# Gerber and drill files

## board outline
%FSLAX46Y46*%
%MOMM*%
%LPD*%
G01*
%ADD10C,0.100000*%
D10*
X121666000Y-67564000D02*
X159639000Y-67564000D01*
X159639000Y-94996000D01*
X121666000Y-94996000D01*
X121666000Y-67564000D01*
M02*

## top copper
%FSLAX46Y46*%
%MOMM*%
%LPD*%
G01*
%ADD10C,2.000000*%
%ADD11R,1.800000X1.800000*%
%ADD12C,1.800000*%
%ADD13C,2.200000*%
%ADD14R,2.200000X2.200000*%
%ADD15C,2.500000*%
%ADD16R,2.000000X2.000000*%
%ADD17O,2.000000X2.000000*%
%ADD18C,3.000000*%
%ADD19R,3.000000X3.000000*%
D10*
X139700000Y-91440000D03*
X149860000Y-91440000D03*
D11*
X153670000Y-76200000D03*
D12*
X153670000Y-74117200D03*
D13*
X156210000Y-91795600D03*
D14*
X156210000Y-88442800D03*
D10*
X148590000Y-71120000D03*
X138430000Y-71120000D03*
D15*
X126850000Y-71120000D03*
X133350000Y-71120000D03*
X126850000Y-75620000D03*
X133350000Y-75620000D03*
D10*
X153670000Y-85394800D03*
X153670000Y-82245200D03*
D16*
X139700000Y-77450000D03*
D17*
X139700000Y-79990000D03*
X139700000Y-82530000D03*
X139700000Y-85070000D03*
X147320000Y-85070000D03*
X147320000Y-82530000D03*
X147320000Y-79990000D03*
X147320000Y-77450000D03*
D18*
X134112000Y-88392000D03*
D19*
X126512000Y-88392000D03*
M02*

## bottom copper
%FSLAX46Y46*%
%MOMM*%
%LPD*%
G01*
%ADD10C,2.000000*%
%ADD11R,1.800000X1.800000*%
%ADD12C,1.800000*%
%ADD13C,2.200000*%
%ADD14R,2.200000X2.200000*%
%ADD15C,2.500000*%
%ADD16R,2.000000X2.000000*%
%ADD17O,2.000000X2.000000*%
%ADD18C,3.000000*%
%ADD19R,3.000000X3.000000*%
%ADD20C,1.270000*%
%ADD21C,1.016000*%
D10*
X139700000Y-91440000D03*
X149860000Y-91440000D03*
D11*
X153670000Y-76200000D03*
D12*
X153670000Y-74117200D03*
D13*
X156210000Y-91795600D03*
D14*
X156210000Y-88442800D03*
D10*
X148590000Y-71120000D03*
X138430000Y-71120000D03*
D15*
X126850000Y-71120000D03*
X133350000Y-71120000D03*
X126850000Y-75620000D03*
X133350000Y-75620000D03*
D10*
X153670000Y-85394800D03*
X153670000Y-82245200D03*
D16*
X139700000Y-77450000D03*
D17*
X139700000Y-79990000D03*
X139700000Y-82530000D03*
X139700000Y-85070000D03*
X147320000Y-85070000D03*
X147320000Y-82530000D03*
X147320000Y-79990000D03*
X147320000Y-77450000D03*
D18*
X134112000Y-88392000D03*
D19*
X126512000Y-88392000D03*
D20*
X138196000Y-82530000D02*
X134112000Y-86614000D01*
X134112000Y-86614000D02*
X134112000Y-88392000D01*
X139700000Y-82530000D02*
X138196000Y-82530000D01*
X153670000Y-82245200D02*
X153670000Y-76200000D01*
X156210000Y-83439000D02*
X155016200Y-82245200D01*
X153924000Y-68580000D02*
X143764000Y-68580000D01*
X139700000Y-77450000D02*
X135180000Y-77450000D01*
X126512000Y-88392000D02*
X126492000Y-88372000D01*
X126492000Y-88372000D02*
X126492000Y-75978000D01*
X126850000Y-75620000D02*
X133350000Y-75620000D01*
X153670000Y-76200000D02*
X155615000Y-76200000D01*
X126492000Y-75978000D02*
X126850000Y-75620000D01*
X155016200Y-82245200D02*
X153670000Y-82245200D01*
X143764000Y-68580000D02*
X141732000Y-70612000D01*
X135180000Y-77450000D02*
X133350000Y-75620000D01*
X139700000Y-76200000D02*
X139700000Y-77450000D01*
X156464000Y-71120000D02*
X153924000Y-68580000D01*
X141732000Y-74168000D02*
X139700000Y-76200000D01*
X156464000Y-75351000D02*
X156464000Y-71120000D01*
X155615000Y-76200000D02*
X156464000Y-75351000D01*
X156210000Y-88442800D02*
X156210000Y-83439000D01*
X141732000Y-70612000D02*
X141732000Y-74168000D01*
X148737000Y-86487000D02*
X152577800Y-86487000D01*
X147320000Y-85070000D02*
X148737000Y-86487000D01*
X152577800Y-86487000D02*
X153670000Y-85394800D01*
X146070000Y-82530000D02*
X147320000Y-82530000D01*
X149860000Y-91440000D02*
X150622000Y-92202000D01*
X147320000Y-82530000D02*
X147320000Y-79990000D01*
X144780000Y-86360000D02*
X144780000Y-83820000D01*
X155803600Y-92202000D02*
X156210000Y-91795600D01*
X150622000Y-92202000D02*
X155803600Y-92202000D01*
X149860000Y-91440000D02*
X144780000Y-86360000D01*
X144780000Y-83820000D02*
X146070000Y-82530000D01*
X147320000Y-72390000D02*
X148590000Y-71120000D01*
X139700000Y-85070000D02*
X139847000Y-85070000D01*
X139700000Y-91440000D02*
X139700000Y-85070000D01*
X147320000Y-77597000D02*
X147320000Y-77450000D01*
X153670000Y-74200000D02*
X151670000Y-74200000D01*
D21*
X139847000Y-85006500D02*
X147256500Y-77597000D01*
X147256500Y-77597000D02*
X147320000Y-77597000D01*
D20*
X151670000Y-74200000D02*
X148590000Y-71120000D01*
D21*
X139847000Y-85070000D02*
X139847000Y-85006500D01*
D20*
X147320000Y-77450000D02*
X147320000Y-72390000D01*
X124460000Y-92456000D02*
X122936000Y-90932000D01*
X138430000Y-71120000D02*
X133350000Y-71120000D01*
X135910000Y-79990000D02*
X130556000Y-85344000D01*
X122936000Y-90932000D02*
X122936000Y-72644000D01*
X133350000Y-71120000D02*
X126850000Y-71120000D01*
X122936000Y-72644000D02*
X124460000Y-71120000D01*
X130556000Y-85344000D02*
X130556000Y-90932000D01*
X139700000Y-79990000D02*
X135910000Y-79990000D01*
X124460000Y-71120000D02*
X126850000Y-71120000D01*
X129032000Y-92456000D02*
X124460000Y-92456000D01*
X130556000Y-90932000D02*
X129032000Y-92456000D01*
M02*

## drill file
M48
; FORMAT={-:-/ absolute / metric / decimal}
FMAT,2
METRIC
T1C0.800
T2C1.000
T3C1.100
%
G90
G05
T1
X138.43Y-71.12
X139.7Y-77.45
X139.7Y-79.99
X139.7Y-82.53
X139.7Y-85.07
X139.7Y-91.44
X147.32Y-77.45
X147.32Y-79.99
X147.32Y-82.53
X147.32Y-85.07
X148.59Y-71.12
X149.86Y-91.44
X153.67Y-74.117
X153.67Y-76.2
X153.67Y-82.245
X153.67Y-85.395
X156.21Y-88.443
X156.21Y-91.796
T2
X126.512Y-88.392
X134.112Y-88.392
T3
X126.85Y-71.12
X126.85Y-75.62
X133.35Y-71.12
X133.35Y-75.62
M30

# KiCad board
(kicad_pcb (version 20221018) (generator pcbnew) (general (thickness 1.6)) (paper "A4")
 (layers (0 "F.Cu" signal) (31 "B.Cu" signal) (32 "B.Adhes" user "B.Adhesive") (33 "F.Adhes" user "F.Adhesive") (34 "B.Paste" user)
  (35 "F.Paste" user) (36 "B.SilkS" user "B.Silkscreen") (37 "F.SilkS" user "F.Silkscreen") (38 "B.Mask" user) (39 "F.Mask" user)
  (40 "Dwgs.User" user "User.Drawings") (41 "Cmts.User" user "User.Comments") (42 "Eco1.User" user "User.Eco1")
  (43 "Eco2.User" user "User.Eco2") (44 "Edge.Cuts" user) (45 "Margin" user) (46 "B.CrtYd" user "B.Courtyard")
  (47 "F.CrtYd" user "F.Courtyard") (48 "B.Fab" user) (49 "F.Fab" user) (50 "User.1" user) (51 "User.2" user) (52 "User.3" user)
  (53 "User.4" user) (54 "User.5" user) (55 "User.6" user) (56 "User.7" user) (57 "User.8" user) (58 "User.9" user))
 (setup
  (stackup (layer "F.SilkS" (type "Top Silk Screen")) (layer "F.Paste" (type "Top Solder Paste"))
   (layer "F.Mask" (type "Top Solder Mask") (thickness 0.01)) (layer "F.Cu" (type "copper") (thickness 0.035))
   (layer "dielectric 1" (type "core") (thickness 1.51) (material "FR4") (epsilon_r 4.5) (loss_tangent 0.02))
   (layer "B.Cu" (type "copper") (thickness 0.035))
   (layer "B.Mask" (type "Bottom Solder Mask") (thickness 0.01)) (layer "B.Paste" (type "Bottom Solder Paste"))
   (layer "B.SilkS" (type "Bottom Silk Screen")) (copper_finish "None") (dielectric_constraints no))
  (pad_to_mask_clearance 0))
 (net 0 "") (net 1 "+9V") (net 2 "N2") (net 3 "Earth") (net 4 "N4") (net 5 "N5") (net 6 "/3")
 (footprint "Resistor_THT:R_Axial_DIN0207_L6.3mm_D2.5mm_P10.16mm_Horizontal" (layer "F.Cu") (at 139.7 91.44)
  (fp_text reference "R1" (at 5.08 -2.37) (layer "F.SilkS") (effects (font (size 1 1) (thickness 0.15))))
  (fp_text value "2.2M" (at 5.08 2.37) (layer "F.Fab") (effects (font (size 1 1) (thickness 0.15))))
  (pad "1" thru_hole circle (at 0 0) (size 2 2) (drill 0.8) (layers "*.Cu" "*.Mask") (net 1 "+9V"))
  (pad "2" thru_hole circle (at 10.16 0) (size 2 2) (drill 0.8) (layers "*.Cu" "*.Mask") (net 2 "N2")))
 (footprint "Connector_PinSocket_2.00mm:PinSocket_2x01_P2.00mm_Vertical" (layer "F.Cu") (at 153.67 76.2 -90)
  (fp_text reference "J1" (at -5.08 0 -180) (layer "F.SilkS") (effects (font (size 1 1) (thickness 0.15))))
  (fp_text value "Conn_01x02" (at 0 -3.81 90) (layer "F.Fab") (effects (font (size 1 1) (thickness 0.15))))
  (pad "1" thru_hole rect (at 0 0 270) (size 1.8 1.8) (drill 0.8) (layers "*.Cu" "*.Mask") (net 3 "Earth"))
  (pad "2" thru_hole circle (at -2.0828 0 270) (size 1.8 1.8) (drill 0.8) (layers "*.Cu" "*.Mask") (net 1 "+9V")))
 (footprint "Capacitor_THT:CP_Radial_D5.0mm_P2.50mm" (layer "F.Cu") (at 156.21 91.44 90)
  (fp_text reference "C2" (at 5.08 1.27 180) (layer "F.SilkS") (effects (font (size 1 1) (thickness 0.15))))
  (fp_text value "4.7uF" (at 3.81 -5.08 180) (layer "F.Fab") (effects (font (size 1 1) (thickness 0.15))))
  (pad "1" thru_hole circle (at -0.3556 0 90) (size 2.2 2.2) (drill 0.8) (layers "*.Cu" "*.Mask") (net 2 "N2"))
  (pad "2" thru_hole rect (at 2.9972 0 90) (size 2.2 2.2) (drill 0.8) (layers "*.Cu" "*.Mask") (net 3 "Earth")))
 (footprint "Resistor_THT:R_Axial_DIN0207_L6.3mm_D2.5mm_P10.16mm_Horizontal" (layer "F.Cu") (at 148.59 71.12 180)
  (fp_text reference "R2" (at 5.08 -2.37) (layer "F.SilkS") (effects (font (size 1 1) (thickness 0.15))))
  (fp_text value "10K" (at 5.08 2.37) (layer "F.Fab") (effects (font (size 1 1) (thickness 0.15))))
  (pad "1" thru_hole circle (at 0 0 180) (size 2 2) (drill 0.8) (layers "*.Cu" "*.Mask") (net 1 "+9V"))
  (pad "2" thru_hole circle (at 10.16 0 180) (size 2 2) (drill 0.8) (layers "*.Cu" "*.Mask") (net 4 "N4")))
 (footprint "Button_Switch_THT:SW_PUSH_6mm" (layer "F.Cu") (at 126.85 71.12)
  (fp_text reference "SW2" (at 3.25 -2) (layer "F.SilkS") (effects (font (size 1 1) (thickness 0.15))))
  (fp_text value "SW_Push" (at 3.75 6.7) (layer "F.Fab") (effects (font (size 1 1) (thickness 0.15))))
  (pad "1" thru_hole circle (at 0 0 90) (size 2.5 2.5) (drill 1.1) (layers "*.Cu" "*.Mask") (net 4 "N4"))
  (pad "1" thru_hole circle (at 6.5 0 90) (size 2.5 2.5) (drill 1.1) (layers "*.Cu" "*.Mask") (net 4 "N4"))
  (pad "2" thru_hole circle (at 0 4.5 90) (size 2.5 2.5) (drill 1.1) (layers "*.Cu" "*.Mask") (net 3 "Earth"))
  (pad "2" thru_hole circle (at 6.5 4.5 90) (size 2.5 2.5) (drill 1.1) (layers "*.Cu" "*.Mask") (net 3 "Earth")))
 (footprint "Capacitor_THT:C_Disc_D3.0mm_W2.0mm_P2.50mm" (layer "F.Cu") (at 153.67 85.09 90)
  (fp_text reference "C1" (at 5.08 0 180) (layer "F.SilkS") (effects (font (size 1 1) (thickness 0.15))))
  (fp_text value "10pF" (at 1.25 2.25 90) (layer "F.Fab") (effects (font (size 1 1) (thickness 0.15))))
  (pad "1" thru_hole circle (at -0.3048 0 90) (size 2 2) (drill 0.8) (layers "*.Cu" "*.Mask") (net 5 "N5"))
  (pad "2" thru_hole circle (at 2.8448 0 90) (size 2 2) (drill 0.8) (layers "*.Cu" "*.Mask") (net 3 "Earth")))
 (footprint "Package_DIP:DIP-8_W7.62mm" (layer "F.Cu") (at 139.7 77.45)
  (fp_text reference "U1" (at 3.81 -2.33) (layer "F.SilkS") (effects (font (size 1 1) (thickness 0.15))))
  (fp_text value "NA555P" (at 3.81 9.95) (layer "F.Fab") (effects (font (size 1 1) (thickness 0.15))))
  (pad "1" thru_hole rect (at 0 0) (size 2 2) (drill 0.8) (layers "*.Cu" "*.Mask") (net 3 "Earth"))
  (pad "2" thru_hole oval (at 0 2.54) (size 2 2) (drill 0.8) (layers "*.Cu" "*.Mask") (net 4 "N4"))
  (pad "3" thru_hole oval (at 0 5.08) (size 2 2) (drill 0.8) (layers "*.Cu" "*.Mask") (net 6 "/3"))
  (pad "4" thru_hole oval (at 0 7.62) (size 2 2) (drill 0.8) (layers "*.Cu" "*.Mask") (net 1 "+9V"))
  (pad "5" thru_hole oval (at 7.62 7.62) (size 2 2) (drill 0.8) (layers "*.Cu" "*.Mask") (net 5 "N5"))
  (pad "6" thru_hole oval (at 7.62 5.08) (size 2 2) (drill 0.8) (layers "*.Cu" "*.Mask") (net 2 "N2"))
  (pad "7" thru_hole oval (at 7.62 2.54) (size 2 2) (drill 0.8) (layers "*.Cu" "*.Mask") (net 2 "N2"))
  (pad "8" thru_hole oval (at 7.62 0) (size 2 2) (drill 0.8) (layers "*.Cu" "*.Mask") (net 1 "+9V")))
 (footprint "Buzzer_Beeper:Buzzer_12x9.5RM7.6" (layer "F.Cu") (at 134.112 88.392 180)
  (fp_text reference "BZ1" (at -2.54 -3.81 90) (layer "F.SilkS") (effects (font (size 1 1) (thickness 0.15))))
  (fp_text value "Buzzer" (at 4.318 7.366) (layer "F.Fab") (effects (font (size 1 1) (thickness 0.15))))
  (pad "1" thru_hole circle (at 0 0 180) (size 3 3) (drill 1) (layers "*.Cu" "*.Mask") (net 6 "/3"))
  (pad "2" thru_hole rect (at 7.6 0 180) (size 3 3) (drill 1) (layers "*.Cu" "*.Mask") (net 3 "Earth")))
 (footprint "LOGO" (layer "B.Cu") (at 150.368 80.899 180)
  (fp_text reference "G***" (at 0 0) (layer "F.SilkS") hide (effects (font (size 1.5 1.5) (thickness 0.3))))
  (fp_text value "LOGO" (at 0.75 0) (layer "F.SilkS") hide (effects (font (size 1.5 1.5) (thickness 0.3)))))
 (gr_rect (start 121.666 67.564) (end 159.639 94.996) (stroke (width 0.1) (type default)) (fill none) (layer "Edge.Cuts"))
 (segment (start 138.196 82.53) (end 134.112 86.614) (width 1.27) (layer "B.Cu") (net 6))
 (segment (start 134.112 86.614) (end 134.112 88.392) (width 1.27) (layer "B.Cu") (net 6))
 (segment (start 139.7 82.53) (end 138.196 82.53) (width 1.27) (layer "B.Cu") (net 6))
 (segment (start 153.67 82.2452) (end 153.67 76.2) (width 1.27) (layer "B.Cu") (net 3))
 (segment (start 156.21 83.439) (end 155.0162 82.2452) (width 1.27) (layer "B.Cu") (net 3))
 (segment (start 153.924 68.58) (end 143.764 68.58) (width 1.27) (layer "B.Cu") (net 3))
 (segment (start 139.7 77.45) (end 135.18 77.45) (width 1.27) (layer "B.Cu") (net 3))
 (segment (start 126.512 88.392) (end 126.492 88.372) (width 1.27) (layer "B.Cu") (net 3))
 (segment (start 126.492 88.372) (end 126.492 75.978) (width 1.27) (layer "B.Cu") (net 3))
 (segment (start 126.85 75.62) (end 133.35 75.62) (width 1.27) (layer "B.Cu") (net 3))
 (segment (start 153.67 76.2) (end 155.615 76.2) (width 1.27) (layer "B.Cu") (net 3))
 (segment (start 126.492 75.978) (end 126.85 75.62) (width 1.27) (layer "B.Cu") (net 3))
 (segment (start 155.0162 82.2452) (end 153.67 82.2452) (width 1.27) (layer "B.Cu") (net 3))
 (segment (start 143.764 68.58) (end 141.732 70.612) (width 1.27) (layer "B.Cu") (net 3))
 (segment (start 135.18 77.45) (end 133.35 75.62) (width 1.27) (layer "B.Cu") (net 3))
 (segment (start 139.7 76.2) (end 139.7 77.45) (width 1.27) (layer "B.Cu") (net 3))
 (segment (start 156.464 71.12) (end 153.924 68.58) (width 1.27) (layer "B.Cu") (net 3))
 (segment (start 141.732 74.168) (end 139.7 76.2) (width 1.27) (layer "B.Cu") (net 3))
 (segment (start 156.464 75.351) (end 156.464 71.12) (width 1.27) (layer "B.Cu") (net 3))
 (segment (start 155.615 76.2) (end 156.464 75.351) (width 1.27) (layer "B.Cu") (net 3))
 (segment (start 156.21 88.4428) (end 156.21 83.439) (width 1.27) (layer "B.Cu") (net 3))
 (segment (start 141.732 70.612) (end 141.732 74.168) (width 1.27) (layer "B.Cu") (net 3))
 (segment (start 148.737 86.487) (end 152.5778 86.487) (width 1.27) (layer "B.Cu") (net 5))
 (segment (start 147.32 85.07) (end 148.737 86.487) (width 1.27) (layer "B.Cu") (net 5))
 (segment (start 152.5778 86.487) (end 153.67 85.3948) (width 1.27) (layer "B.Cu") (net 5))
 (segment (start 146.07 82.53) (end 147.32 82.53) (width 1.27) (layer "B.Cu") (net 2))
 (segment (start 149.86 91.44) (end 150.622 92.202) (width 1.27) (layer "B.Cu") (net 2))
 (segment (start 147.32 82.53) (end 147.32 79.99) (width 1.27) (layer "B.Cu") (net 2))
 (segment (start 144.78 86.36) (end 144.78 83.82) (width 1.27) (layer "B.Cu") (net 2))
 (segment (start 155.8036 92.202) (end 156.21 91.7956) (width 1.27) (layer "B.Cu") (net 2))
 (segment (start 150.622 92.202) (end 155.8036 92.202) (width 1.27) (layer "B.Cu") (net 2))
 (segment (start 149.86 91.44) (end 144.78 86.36) (width 1.27) (layer "B.Cu") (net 2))
 (segment (start 144.78 83.82) (end 146.07 82.53) (width 1.27) (layer "B.Cu") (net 2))
 (segment (start 147.32 72.39) (end 148.59 71.12) (width 1.27) (layer "B.Cu") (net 1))
 (segment (start 139.7 85.07) (end 139.847 85.07) (width 1.27) (layer "B.Cu") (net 1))
 (segment (start 139.7 91.44) (end 139.7 85.07) (width 1.27) (layer "B.Cu") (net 1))
 (segment (start 147.32 77.597) (end 147.32 77.45) (width 1.27) (layer "B.Cu") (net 1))
 (segment (start 153.67 74.2) (end 151.67 74.2) (width 1.27) (layer "B.Cu") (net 1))
 (segment (start 139.847 85.0065) (end 147.2565 77.597) (width 1.016) (layer "B.Cu") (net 1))
 (segment (start 147.2565 77.597) (end 147.32 77.597) (width 1.016) (layer "B.Cu") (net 1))
 (segment (start 151.67 74.2) (end 148.59 71.12) (width 1.27) (layer "B.Cu") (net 1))
 (segment (start 139.847 85.07) (end 139.847 85.0065) (width 1.016) (layer "B.Cu") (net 1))
 (segment (start 147.32 77.45) (end 147.32 72.39) (width 1.27) (layer "B.Cu") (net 1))
 (segment (start 124.46 92.456) (end 122.936 90.932) (width 1.27) (layer "B.Cu") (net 4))
 (segment (start 138.43 71.12) (end 133.35 71.12) (width 1.27) (layer "B.Cu") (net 4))
 (segment (start 135.91 79.99) (end 130.556 85.344) (width 1.27) (layer "B.Cu") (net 4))
 (segment (start 122.936 90.932) (end 122.936 72.644) (width 1.27) (layer "B.Cu") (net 4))
 (segment (start 133.35 71.12) (end 126.85 71.12) (width 1.27) (layer "B.Cu") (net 4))
 (segment (start 122.936 72.644) (end 124.46 71.12) (width 1.27) (layer "B.Cu") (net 4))
 (segment (start 130.556 85.344) (end 130.556 90.932) (width 1.27) (layer "B.Cu") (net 4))
 (segment (start 139.7 79.99) (end 135.91 79.99) (width 1.27) (layer "B.Cu") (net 4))
 (segment (start 124.46 71.12) (end 126.85 71.12) (width 1.27) (layer "B.Cu") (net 4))
 (segment (start 129.032 92.456) (end 124.46 92.456) (width 1.27) (layer "B.Cu") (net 4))
 (segment (start 130.556 90.932) (end 129.032 92.456) (width 1.27) (layer "B.Cu") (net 4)))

